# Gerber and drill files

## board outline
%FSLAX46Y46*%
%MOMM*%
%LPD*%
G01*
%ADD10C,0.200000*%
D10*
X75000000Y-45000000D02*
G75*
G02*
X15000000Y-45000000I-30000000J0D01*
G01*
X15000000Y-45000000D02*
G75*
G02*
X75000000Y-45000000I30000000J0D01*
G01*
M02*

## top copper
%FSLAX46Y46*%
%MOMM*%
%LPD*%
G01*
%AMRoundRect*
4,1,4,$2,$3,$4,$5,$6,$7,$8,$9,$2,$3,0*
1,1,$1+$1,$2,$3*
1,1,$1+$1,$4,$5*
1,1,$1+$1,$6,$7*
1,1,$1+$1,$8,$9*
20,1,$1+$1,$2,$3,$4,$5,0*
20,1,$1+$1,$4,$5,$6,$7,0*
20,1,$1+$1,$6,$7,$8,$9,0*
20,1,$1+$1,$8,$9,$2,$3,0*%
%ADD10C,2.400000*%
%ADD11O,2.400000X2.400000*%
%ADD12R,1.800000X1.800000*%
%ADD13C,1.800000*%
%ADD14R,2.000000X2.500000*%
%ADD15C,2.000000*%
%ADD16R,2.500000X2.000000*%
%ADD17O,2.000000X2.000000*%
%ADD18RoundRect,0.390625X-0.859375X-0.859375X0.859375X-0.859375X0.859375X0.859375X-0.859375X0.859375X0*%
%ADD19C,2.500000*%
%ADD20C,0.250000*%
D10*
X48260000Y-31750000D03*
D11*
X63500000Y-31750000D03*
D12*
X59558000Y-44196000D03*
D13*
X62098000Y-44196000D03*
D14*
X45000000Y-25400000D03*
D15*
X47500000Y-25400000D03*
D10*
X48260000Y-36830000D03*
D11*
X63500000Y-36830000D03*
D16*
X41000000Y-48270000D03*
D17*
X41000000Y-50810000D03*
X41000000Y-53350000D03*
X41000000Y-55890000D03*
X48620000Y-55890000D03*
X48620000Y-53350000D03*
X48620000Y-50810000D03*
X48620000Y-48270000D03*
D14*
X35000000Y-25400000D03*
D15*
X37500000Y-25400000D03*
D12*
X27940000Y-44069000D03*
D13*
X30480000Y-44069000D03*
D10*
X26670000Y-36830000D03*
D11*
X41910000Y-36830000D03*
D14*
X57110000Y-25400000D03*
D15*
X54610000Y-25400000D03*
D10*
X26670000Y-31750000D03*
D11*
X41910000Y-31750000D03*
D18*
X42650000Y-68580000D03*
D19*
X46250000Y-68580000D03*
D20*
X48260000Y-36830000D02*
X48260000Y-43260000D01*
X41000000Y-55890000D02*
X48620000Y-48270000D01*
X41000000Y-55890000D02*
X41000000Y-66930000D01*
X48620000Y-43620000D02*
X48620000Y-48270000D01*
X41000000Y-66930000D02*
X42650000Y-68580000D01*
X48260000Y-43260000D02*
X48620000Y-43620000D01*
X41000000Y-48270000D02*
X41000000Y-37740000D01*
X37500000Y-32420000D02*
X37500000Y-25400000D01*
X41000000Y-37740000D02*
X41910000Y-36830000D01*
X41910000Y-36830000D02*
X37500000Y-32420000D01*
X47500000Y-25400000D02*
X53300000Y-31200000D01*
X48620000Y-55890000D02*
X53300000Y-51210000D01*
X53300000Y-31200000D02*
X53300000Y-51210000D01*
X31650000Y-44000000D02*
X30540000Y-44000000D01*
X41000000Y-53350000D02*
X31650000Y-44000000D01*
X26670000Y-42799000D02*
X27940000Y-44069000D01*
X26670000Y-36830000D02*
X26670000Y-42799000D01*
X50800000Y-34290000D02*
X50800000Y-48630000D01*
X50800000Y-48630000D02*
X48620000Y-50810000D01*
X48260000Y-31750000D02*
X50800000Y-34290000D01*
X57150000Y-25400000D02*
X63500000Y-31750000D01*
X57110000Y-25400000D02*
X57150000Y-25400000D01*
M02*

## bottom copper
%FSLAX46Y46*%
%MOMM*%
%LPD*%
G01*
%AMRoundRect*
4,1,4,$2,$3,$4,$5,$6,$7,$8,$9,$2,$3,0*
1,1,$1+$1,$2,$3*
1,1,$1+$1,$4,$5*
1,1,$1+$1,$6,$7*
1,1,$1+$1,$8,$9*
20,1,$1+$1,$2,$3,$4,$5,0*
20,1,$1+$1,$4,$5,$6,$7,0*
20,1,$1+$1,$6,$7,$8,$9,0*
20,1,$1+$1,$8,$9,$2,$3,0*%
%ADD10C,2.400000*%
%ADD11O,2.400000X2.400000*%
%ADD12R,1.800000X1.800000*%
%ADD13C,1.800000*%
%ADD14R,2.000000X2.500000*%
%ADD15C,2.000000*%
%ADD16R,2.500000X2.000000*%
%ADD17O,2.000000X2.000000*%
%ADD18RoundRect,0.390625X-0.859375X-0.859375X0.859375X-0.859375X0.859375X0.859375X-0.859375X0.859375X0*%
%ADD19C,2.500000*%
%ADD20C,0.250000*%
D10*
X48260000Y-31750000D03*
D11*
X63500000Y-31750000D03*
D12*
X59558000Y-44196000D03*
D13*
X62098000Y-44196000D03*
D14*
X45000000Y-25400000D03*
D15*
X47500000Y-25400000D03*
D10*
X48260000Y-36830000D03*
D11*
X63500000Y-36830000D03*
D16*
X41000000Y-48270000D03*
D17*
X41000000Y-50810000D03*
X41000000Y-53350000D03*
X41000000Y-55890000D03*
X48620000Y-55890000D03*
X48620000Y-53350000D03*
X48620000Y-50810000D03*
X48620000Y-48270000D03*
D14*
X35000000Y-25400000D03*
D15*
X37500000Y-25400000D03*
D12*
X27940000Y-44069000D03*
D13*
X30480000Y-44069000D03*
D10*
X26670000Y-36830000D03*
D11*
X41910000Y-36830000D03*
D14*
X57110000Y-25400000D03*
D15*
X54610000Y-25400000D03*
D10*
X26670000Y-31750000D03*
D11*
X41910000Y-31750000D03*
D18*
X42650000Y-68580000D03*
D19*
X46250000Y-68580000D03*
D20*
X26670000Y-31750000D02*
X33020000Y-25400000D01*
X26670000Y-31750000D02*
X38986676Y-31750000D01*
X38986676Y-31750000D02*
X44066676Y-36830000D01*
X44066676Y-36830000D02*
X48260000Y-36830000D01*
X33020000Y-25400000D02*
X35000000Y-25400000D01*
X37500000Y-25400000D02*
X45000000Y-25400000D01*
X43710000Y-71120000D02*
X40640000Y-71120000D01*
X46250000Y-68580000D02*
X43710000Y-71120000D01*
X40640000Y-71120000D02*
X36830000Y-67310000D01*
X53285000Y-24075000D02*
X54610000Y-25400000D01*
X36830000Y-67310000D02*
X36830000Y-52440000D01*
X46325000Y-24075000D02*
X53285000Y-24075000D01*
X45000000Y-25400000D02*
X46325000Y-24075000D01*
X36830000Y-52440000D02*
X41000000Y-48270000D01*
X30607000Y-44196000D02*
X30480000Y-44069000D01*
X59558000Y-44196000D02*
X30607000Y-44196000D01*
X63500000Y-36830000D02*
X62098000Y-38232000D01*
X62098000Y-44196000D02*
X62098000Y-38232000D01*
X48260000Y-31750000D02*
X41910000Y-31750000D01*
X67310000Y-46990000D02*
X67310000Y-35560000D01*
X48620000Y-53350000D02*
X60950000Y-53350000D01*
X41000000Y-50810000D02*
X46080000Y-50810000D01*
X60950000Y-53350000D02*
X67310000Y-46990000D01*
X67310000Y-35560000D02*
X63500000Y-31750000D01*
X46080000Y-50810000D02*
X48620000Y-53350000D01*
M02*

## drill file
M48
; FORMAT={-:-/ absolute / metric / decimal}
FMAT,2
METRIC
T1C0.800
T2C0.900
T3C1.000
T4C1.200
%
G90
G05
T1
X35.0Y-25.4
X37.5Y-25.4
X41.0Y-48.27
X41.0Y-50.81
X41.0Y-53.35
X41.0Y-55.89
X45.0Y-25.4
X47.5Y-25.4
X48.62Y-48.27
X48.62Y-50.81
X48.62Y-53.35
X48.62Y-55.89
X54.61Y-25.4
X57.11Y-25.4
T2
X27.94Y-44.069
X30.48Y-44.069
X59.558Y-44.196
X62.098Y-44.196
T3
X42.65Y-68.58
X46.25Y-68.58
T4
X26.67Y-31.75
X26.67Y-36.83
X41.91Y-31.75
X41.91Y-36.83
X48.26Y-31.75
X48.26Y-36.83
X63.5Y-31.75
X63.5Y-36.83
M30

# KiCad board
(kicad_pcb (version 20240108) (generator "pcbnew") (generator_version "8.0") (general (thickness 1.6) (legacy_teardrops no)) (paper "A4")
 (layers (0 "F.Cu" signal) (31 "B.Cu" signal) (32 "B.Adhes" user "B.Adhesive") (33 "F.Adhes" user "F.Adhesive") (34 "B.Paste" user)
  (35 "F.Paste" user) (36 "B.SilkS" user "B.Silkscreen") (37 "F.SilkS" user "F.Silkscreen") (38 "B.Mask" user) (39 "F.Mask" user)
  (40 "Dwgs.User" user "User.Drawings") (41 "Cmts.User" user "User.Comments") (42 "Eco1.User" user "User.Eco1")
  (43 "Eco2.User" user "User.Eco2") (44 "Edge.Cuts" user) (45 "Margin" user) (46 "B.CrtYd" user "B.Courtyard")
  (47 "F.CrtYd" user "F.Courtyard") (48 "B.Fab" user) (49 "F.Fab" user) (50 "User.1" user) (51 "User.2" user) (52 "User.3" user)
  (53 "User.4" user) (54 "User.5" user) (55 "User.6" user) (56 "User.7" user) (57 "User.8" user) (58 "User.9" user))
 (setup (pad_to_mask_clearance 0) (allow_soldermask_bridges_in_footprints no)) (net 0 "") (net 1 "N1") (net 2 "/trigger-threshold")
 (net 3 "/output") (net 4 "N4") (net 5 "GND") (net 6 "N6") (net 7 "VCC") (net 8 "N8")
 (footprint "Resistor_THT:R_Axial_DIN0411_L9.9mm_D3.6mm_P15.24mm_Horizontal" (layer "F.Cu") (at 48.26 31.75)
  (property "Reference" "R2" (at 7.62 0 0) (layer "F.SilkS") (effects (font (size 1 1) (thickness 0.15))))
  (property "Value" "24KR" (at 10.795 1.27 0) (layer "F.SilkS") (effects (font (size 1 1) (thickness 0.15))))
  (pad "1" thru_hole circle (at 0 0) (size 2.4 2.4) (drill 1.2) (layers "*.Cu" "*.Mask") (remove_unused_layers no) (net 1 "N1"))
  (pad "2" thru_hole oval (at 15.24 0) (size 2.4 2.4) (drill 1.2) (layers "*.Cu" "*.Mask") (remove_unused_layers no)
   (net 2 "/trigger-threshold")))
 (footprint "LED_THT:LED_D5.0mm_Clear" (layer "F.Cu") (at 59.558 44.196)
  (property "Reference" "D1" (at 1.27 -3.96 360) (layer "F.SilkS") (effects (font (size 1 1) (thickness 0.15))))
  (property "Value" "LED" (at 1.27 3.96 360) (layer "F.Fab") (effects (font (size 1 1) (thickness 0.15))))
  (pad "1" thru_hole rect (at 0 0) (size 1.8 1.8) (drill 0.9) (layers "*.Cu" "*.Mask") (remove_unused_layers no) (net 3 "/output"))
  (pad "2" thru_hole circle (at 2.54 0) (size 1.8 1.8) (drill 0.9) (layers "*.Cu" "*.Mask") (remove_unused_layers no) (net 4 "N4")))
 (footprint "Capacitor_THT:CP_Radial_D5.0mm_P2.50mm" (layer "F.Cu") (at 45 25.4)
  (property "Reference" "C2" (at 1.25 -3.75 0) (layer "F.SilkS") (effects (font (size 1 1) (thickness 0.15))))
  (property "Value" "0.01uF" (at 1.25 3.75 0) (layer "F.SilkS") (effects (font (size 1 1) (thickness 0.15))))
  (pad "1" thru_hole rect (at 0 0) (size 2 2.5) (drill 0.8) (layers "*.Cu" "*.Mask") (remove_unused_layers no) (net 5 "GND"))
  (pad "2" thru_hole circle (at 2.5 0) (size 2 2) (drill 0.8) (layers "*.Cu" "*.Mask") (remove_unused_layers no) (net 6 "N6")))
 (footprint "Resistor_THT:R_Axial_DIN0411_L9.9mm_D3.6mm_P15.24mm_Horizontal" (layer "F.Cu") (at 48.26 36.83)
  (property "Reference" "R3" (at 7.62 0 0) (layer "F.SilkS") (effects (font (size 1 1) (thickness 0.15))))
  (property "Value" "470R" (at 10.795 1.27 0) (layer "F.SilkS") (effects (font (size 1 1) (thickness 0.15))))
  (pad "1" thru_hole circle (at 0 0) (size 2.4 2.4) (drill 1.2) (layers "*.Cu" "*.Mask") (remove_unused_layers no) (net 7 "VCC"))
  (pad "2" thru_hole oval (at 15.24 0) (size 2.4 2.4) (drill 1.2) (layers "*.Cu" "*.Mask") (remove_unused_layers no) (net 4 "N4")))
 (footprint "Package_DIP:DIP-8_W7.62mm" (layer "F.Cu") (at 41 48.27)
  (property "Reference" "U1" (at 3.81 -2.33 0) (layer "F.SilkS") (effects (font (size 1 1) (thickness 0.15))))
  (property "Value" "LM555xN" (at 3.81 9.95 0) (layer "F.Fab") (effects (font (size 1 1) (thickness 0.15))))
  (pad "1" thru_hole rect (at 0 0) (size 2.5 2) (drill 0.8) (layers "*.Cu" "*.Mask") (remove_unused_layers no) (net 5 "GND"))
  (pad "2" thru_hole oval (at 0 2.54) (size 2 2) (drill 0.8) (layers "*.Cu" "*.Mask") (remove_unused_layers no) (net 2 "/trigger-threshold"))
  (pad "3" thru_hole oval (at 0 5.08) (size 2 2) (drill 0.8) (layers "*.Cu" "*.Mask") (remove_unused_layers no) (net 3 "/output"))
  (pad "4" thru_hole oval (at 0 7.62) (size 2 2) (drill 0.8) (layers "*.Cu" "*.Mask") (remove_unused_layers no) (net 7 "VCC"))
  (pad "5" thru_hole oval (at 7.62 7.62) (size 2 2) (drill 0.8) (layers "*.Cu" "*.Mask") (remove_unused_layers no) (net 6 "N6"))
  (pad "6" thru_hole oval (at 7.62 5.08) (size 2 2) (drill 0.8) (layers "*.Cu" "*.Mask") (remove_unused_layers no)
   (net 2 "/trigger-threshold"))
  (pad "7" thru_hole oval (at 7.62 2.54) (size 2 2) (drill 0.8) (layers "*.Cu" "*.Mask") (remove_unused_layers no) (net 1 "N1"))
  (pad "8" thru_hole oval (at 7.62 0) (size 2 2) (drill 0.8) (layers "*.Cu" "*.Mask") (remove_unused_layers no) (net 7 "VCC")))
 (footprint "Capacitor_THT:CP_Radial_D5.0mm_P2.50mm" (layer "F.Cu") (at 35 25.4)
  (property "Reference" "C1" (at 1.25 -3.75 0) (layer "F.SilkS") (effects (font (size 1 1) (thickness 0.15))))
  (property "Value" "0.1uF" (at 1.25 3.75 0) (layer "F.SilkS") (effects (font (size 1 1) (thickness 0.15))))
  (pad "1" thru_hole rect (at 0 0) (size 2 2.5) (drill 0.8) (layers "*.Cu" "*.Mask") (remove_unused_layers no) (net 7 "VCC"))
  (pad "2" thru_hole circle (at 2.5 0) (size 2 2) (drill 0.8) (layers "*.Cu" "*.Mask") (remove_unused_layers no) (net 5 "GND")))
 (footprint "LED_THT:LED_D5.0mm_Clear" (layer "F.Cu") (at 27.94 44.069)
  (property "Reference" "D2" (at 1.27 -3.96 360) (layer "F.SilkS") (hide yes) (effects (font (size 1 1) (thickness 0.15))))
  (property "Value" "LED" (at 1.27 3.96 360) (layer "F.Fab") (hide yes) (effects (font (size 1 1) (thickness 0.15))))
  (pad "1" thru_hole rect (at 0 0) (size 1.8 1.8) (drill 0.9) (layers "*.Cu" "*.Mask") (remove_unused_layers no) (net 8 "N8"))
  (pad "2" thru_hole circle (at 2.54 0) (size 1.8 1.8) (drill 0.9) (layers "*.Cu" "*.Mask") (remove_unused_layers no) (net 3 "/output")))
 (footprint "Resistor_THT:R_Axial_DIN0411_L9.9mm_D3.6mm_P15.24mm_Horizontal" (layer "F.Cu") (at 26.67 36.83)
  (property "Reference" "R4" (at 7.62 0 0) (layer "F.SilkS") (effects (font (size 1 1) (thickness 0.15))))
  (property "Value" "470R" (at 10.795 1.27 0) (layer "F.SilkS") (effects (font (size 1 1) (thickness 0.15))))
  (pad "1" thru_hole circle (at 0 0) (size 2.4 2.4) (drill 1.2) (layers "*.Cu" "*.Mask") (remove_unused_layers no) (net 8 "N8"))
  (pad "2" thru_hole oval (at 15.24 0) (size 2.4 2.4) (drill 1.2) (layers "*.Cu" "*.Mask") (remove_unused_layers no) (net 5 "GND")))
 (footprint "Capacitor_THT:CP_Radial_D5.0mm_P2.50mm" (layer "F.Cu") (at 57.11 25.4 180)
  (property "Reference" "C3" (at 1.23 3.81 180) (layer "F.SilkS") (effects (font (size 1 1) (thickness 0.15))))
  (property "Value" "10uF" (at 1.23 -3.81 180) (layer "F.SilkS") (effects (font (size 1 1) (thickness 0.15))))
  (pad "1" thru_hole rect (at 0 0 180) (size 2 2.5) (drill 0.8) (layers "*.Cu" "*.Mask") (remove_unused_layers no)
   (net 2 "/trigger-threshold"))
  (pad "2" thru_hole circle (at 2.5 0 180) (size 2 2) (drill 0.8) (layers "*.Cu" "*.Mask") (remove_unused_layers no) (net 5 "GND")))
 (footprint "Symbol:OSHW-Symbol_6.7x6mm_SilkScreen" (layer "F.Cu") (at 45.085 41.91)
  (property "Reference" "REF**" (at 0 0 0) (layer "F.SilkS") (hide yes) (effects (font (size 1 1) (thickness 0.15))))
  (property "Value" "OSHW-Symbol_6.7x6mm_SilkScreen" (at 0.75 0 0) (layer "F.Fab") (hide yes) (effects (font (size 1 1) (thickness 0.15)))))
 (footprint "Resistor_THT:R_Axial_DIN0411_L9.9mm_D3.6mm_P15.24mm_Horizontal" (layer "F.Cu") (at 26.67 31.75)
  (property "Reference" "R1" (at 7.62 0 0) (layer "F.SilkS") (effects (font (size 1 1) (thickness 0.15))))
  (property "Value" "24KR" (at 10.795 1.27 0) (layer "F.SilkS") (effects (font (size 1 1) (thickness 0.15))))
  (pad "1" thru_hole circle (at 0 0) (size 2.4 2.4) (drill 1.2) (layers "*.Cu" "*.Mask") (remove_unused_layers no) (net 7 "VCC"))
  (pad "2" thru_hole oval (at 15.24 0) (size 2.4 2.4) (drill 1.2) (layers "*.Cu" "*.Mask") (remove_unused_layers no) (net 1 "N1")))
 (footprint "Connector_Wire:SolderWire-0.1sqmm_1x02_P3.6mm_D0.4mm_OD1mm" (layer "F.Cu") (at 42.65 68.58)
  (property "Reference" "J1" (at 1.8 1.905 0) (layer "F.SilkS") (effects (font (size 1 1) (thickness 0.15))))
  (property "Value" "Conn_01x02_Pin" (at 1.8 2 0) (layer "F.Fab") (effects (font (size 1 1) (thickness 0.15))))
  (pad "1" thru_hole roundrect (at 0 0) (size 2.5 2.5) (drill 1) (layers "*.Cu" "*.Mask") (remove_unused_layers no)
   (roundrect_rratio 0.15625) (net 7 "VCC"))
  (pad "2" thru_hole circle (at 3.6 0) (size 2.5 2.5) (drill 1) (layers "*.Cu" "*.Mask") (remove_unused_layers no) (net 5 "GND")))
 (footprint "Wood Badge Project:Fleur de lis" (layer "B.Cu") (at 45 45 180)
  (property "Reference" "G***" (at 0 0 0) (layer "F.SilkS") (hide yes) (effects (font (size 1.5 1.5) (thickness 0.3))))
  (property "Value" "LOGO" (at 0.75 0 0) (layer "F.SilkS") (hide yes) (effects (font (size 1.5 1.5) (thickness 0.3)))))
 (gr_circle (center 45 45) (end 75 45) (stroke (width 0.2) (type default)) (fill none) (layer "Edge.Cuts"))
 (segment (start 48.26 36.83) (end 48.26 43.26) (width 0.25) (layer "F.Cu") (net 7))
 (segment (start 41 55.89) (end 48.62 48.27) (width 0.25) (layer "F.Cu") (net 7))
 (segment (start 41 55.89) (end 41 66.93) (width 0.25) (layer "F.Cu") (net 7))
 (segment (start 48.62 43.62) (end 48.62 48.27) (width 0.25) (layer "F.Cu") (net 7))
 (segment (start 41 66.93) (end 42.65 68.58) (width 0.25) (layer "F.Cu") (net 7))
 (segment (start 48.26 43.26) (end 48.62 43.62) (width 0.25) (layer "F.Cu") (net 7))
 (segment (start 26.67 31.75) (end 33.02 25.4) (width 0.25) (layer "B.Cu") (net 7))
 (segment (start 26.67 31.75) (end 38.986676 31.75) (width 0.25) (layer "B.Cu") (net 7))
 (segment (start 38.986676 31.75) (end 44.066676 36.83) (width 0.25) (layer "B.Cu") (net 7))
 (segment (start 44.066676 36.83) (end 48.26 36.83) (width 0.25) (layer "B.Cu") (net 7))
 (segment (start 33.02 25.4) (end 35 25.4) (width 0.25) (layer "B.Cu") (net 7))
 (segment (start 41 48.27) (end 41 37.74) (width 0.25) (layer "F.Cu") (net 5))
 (segment (start 37.5 32.42) (end 37.5 25.4) (width 0.25) (layer "F.Cu") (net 5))
 (segment (start 41 37.74) (end 41.91 36.83) (width 0.25) (layer "F.Cu") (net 5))
 (segment (start 41.91 36.83) (end 37.5 32.42) (width 0.25) (layer "F.Cu") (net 5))
 (segment (start 37.5 25.4) (end 45 25.4) (width 0.25) (layer "B.Cu") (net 5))
 (segment (start 43.71 71.12) (end 40.64 71.12) (width 0.25) (layer "B.Cu") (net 5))
 (segment (start 46.25 68.58) (end 43.71 71.12) (width 0.25) (layer "B.Cu") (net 5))
 (segment (start 40.64 71.12) (end 36.83 67.31) (width 0.25) (layer "B.Cu") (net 5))
 (segment (start 53.285 24.075) (end 54.61 25.4) (width 0.25) (layer "B.Cu") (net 5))
 (segment (start 36.83 67.31) (end 36.83 52.44) (width 0.25) (layer "B.Cu") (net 5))
 (segment (start 46.325 24.075) (end 53.285 24.075) (width 0.25) (layer "B.Cu") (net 5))
 (segment (start 45 25.4) (end 46.325 24.075) (width 0.25) (layer "B.Cu") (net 5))
 (segment (start 36.83 52.44) (end 41 48.27) (width 0.25) (layer "B.Cu") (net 5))
 (segment (start 47.5 25.4) (end 53.3 31.2) (width 0.25) (layer "F.Cu") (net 6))
 (segment (start 48.62 55.89) (end 53.3 51.21) (width 0.25) (layer "F.Cu") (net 6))
 (segment (start 53.3 31.2) (end 53.3 51.21) (width 0.25) (layer "F.Cu") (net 6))
 (segment (start 31.65 44) (end 30.54 44) (width 0.25) (layer "F.Cu") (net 3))
 (segment (start 41 53.35) (end 31.65 44) (width 0.25) (layer "F.Cu") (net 3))
 (segment (start 30.607 44.196) (end 30.48 44.069) (width 0.25) (layer "B.Cu") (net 3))
 (segment (start 59.558 44.196) (end 30.607 44.196) (width 0.25) (layer "B.Cu") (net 3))
 (segment (start 63.5 36.83) (end 62.098 38.232) (width 0.25) (layer "B.Cu") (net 4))
 (segment (start 62.098 44.196) (end 62.098 38.232) (width 0.25) (layer "B.Cu") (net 4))
 (segment (start 26.67 42.799) (end 27.94 44.069) (width 0.25) (layer "F.Cu") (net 8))
 (segment (start 26.67 36.83) (end 26.67 42.799) (width 0.25) (layer "F.Cu") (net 8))
 (segment (start 50.8 34.29) (end 50.8 48.63) (width 0.25) (layer "F.Cu") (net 1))
 (segment (start 50.8 48.63) (end 48.62 50.81) (width 0.25) (layer "F.Cu") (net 1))
 (segment (start 48.26 31.75) (end 50.8 34.29) (width 0.25) (layer "F.Cu") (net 1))
 (segment (start 48.26 31.75) (end 41.91 31.75) (width 0.25) (layer "B.Cu") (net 1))
 (segment (start 57.15 25.4) (end 63.5 31.75) (width 0.25) (layer "F.Cu") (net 2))
 (segment (start 57.11 25.4) (end 57.15 25.4) (width 0.25) (layer "F.Cu") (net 2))
 (segment (start 67.31 46.99) (end 67.31 35.56) (width 0.25) (layer "B.Cu") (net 2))
 (segment (start 48.62 53.35) (end 60.95 53.35) (width 0.25) (layer "B.Cu") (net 2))
 (segment (start 41 50.81) (end 46.08 50.81) (width 0.25) (layer "B.Cu") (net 2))
 (segment (start 60.95 53.35) (end 67.31 46.99) (width 0.25) (layer "B.Cu") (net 2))
 (segment (start 67.31 35.56) (end 63.5 31.75) (width 0.25) (layer "B.Cu") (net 2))
 (segment (start 46.08 50.81) (end 48.62 53.35) (width 0.25) (layer "B.Cu") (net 2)))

